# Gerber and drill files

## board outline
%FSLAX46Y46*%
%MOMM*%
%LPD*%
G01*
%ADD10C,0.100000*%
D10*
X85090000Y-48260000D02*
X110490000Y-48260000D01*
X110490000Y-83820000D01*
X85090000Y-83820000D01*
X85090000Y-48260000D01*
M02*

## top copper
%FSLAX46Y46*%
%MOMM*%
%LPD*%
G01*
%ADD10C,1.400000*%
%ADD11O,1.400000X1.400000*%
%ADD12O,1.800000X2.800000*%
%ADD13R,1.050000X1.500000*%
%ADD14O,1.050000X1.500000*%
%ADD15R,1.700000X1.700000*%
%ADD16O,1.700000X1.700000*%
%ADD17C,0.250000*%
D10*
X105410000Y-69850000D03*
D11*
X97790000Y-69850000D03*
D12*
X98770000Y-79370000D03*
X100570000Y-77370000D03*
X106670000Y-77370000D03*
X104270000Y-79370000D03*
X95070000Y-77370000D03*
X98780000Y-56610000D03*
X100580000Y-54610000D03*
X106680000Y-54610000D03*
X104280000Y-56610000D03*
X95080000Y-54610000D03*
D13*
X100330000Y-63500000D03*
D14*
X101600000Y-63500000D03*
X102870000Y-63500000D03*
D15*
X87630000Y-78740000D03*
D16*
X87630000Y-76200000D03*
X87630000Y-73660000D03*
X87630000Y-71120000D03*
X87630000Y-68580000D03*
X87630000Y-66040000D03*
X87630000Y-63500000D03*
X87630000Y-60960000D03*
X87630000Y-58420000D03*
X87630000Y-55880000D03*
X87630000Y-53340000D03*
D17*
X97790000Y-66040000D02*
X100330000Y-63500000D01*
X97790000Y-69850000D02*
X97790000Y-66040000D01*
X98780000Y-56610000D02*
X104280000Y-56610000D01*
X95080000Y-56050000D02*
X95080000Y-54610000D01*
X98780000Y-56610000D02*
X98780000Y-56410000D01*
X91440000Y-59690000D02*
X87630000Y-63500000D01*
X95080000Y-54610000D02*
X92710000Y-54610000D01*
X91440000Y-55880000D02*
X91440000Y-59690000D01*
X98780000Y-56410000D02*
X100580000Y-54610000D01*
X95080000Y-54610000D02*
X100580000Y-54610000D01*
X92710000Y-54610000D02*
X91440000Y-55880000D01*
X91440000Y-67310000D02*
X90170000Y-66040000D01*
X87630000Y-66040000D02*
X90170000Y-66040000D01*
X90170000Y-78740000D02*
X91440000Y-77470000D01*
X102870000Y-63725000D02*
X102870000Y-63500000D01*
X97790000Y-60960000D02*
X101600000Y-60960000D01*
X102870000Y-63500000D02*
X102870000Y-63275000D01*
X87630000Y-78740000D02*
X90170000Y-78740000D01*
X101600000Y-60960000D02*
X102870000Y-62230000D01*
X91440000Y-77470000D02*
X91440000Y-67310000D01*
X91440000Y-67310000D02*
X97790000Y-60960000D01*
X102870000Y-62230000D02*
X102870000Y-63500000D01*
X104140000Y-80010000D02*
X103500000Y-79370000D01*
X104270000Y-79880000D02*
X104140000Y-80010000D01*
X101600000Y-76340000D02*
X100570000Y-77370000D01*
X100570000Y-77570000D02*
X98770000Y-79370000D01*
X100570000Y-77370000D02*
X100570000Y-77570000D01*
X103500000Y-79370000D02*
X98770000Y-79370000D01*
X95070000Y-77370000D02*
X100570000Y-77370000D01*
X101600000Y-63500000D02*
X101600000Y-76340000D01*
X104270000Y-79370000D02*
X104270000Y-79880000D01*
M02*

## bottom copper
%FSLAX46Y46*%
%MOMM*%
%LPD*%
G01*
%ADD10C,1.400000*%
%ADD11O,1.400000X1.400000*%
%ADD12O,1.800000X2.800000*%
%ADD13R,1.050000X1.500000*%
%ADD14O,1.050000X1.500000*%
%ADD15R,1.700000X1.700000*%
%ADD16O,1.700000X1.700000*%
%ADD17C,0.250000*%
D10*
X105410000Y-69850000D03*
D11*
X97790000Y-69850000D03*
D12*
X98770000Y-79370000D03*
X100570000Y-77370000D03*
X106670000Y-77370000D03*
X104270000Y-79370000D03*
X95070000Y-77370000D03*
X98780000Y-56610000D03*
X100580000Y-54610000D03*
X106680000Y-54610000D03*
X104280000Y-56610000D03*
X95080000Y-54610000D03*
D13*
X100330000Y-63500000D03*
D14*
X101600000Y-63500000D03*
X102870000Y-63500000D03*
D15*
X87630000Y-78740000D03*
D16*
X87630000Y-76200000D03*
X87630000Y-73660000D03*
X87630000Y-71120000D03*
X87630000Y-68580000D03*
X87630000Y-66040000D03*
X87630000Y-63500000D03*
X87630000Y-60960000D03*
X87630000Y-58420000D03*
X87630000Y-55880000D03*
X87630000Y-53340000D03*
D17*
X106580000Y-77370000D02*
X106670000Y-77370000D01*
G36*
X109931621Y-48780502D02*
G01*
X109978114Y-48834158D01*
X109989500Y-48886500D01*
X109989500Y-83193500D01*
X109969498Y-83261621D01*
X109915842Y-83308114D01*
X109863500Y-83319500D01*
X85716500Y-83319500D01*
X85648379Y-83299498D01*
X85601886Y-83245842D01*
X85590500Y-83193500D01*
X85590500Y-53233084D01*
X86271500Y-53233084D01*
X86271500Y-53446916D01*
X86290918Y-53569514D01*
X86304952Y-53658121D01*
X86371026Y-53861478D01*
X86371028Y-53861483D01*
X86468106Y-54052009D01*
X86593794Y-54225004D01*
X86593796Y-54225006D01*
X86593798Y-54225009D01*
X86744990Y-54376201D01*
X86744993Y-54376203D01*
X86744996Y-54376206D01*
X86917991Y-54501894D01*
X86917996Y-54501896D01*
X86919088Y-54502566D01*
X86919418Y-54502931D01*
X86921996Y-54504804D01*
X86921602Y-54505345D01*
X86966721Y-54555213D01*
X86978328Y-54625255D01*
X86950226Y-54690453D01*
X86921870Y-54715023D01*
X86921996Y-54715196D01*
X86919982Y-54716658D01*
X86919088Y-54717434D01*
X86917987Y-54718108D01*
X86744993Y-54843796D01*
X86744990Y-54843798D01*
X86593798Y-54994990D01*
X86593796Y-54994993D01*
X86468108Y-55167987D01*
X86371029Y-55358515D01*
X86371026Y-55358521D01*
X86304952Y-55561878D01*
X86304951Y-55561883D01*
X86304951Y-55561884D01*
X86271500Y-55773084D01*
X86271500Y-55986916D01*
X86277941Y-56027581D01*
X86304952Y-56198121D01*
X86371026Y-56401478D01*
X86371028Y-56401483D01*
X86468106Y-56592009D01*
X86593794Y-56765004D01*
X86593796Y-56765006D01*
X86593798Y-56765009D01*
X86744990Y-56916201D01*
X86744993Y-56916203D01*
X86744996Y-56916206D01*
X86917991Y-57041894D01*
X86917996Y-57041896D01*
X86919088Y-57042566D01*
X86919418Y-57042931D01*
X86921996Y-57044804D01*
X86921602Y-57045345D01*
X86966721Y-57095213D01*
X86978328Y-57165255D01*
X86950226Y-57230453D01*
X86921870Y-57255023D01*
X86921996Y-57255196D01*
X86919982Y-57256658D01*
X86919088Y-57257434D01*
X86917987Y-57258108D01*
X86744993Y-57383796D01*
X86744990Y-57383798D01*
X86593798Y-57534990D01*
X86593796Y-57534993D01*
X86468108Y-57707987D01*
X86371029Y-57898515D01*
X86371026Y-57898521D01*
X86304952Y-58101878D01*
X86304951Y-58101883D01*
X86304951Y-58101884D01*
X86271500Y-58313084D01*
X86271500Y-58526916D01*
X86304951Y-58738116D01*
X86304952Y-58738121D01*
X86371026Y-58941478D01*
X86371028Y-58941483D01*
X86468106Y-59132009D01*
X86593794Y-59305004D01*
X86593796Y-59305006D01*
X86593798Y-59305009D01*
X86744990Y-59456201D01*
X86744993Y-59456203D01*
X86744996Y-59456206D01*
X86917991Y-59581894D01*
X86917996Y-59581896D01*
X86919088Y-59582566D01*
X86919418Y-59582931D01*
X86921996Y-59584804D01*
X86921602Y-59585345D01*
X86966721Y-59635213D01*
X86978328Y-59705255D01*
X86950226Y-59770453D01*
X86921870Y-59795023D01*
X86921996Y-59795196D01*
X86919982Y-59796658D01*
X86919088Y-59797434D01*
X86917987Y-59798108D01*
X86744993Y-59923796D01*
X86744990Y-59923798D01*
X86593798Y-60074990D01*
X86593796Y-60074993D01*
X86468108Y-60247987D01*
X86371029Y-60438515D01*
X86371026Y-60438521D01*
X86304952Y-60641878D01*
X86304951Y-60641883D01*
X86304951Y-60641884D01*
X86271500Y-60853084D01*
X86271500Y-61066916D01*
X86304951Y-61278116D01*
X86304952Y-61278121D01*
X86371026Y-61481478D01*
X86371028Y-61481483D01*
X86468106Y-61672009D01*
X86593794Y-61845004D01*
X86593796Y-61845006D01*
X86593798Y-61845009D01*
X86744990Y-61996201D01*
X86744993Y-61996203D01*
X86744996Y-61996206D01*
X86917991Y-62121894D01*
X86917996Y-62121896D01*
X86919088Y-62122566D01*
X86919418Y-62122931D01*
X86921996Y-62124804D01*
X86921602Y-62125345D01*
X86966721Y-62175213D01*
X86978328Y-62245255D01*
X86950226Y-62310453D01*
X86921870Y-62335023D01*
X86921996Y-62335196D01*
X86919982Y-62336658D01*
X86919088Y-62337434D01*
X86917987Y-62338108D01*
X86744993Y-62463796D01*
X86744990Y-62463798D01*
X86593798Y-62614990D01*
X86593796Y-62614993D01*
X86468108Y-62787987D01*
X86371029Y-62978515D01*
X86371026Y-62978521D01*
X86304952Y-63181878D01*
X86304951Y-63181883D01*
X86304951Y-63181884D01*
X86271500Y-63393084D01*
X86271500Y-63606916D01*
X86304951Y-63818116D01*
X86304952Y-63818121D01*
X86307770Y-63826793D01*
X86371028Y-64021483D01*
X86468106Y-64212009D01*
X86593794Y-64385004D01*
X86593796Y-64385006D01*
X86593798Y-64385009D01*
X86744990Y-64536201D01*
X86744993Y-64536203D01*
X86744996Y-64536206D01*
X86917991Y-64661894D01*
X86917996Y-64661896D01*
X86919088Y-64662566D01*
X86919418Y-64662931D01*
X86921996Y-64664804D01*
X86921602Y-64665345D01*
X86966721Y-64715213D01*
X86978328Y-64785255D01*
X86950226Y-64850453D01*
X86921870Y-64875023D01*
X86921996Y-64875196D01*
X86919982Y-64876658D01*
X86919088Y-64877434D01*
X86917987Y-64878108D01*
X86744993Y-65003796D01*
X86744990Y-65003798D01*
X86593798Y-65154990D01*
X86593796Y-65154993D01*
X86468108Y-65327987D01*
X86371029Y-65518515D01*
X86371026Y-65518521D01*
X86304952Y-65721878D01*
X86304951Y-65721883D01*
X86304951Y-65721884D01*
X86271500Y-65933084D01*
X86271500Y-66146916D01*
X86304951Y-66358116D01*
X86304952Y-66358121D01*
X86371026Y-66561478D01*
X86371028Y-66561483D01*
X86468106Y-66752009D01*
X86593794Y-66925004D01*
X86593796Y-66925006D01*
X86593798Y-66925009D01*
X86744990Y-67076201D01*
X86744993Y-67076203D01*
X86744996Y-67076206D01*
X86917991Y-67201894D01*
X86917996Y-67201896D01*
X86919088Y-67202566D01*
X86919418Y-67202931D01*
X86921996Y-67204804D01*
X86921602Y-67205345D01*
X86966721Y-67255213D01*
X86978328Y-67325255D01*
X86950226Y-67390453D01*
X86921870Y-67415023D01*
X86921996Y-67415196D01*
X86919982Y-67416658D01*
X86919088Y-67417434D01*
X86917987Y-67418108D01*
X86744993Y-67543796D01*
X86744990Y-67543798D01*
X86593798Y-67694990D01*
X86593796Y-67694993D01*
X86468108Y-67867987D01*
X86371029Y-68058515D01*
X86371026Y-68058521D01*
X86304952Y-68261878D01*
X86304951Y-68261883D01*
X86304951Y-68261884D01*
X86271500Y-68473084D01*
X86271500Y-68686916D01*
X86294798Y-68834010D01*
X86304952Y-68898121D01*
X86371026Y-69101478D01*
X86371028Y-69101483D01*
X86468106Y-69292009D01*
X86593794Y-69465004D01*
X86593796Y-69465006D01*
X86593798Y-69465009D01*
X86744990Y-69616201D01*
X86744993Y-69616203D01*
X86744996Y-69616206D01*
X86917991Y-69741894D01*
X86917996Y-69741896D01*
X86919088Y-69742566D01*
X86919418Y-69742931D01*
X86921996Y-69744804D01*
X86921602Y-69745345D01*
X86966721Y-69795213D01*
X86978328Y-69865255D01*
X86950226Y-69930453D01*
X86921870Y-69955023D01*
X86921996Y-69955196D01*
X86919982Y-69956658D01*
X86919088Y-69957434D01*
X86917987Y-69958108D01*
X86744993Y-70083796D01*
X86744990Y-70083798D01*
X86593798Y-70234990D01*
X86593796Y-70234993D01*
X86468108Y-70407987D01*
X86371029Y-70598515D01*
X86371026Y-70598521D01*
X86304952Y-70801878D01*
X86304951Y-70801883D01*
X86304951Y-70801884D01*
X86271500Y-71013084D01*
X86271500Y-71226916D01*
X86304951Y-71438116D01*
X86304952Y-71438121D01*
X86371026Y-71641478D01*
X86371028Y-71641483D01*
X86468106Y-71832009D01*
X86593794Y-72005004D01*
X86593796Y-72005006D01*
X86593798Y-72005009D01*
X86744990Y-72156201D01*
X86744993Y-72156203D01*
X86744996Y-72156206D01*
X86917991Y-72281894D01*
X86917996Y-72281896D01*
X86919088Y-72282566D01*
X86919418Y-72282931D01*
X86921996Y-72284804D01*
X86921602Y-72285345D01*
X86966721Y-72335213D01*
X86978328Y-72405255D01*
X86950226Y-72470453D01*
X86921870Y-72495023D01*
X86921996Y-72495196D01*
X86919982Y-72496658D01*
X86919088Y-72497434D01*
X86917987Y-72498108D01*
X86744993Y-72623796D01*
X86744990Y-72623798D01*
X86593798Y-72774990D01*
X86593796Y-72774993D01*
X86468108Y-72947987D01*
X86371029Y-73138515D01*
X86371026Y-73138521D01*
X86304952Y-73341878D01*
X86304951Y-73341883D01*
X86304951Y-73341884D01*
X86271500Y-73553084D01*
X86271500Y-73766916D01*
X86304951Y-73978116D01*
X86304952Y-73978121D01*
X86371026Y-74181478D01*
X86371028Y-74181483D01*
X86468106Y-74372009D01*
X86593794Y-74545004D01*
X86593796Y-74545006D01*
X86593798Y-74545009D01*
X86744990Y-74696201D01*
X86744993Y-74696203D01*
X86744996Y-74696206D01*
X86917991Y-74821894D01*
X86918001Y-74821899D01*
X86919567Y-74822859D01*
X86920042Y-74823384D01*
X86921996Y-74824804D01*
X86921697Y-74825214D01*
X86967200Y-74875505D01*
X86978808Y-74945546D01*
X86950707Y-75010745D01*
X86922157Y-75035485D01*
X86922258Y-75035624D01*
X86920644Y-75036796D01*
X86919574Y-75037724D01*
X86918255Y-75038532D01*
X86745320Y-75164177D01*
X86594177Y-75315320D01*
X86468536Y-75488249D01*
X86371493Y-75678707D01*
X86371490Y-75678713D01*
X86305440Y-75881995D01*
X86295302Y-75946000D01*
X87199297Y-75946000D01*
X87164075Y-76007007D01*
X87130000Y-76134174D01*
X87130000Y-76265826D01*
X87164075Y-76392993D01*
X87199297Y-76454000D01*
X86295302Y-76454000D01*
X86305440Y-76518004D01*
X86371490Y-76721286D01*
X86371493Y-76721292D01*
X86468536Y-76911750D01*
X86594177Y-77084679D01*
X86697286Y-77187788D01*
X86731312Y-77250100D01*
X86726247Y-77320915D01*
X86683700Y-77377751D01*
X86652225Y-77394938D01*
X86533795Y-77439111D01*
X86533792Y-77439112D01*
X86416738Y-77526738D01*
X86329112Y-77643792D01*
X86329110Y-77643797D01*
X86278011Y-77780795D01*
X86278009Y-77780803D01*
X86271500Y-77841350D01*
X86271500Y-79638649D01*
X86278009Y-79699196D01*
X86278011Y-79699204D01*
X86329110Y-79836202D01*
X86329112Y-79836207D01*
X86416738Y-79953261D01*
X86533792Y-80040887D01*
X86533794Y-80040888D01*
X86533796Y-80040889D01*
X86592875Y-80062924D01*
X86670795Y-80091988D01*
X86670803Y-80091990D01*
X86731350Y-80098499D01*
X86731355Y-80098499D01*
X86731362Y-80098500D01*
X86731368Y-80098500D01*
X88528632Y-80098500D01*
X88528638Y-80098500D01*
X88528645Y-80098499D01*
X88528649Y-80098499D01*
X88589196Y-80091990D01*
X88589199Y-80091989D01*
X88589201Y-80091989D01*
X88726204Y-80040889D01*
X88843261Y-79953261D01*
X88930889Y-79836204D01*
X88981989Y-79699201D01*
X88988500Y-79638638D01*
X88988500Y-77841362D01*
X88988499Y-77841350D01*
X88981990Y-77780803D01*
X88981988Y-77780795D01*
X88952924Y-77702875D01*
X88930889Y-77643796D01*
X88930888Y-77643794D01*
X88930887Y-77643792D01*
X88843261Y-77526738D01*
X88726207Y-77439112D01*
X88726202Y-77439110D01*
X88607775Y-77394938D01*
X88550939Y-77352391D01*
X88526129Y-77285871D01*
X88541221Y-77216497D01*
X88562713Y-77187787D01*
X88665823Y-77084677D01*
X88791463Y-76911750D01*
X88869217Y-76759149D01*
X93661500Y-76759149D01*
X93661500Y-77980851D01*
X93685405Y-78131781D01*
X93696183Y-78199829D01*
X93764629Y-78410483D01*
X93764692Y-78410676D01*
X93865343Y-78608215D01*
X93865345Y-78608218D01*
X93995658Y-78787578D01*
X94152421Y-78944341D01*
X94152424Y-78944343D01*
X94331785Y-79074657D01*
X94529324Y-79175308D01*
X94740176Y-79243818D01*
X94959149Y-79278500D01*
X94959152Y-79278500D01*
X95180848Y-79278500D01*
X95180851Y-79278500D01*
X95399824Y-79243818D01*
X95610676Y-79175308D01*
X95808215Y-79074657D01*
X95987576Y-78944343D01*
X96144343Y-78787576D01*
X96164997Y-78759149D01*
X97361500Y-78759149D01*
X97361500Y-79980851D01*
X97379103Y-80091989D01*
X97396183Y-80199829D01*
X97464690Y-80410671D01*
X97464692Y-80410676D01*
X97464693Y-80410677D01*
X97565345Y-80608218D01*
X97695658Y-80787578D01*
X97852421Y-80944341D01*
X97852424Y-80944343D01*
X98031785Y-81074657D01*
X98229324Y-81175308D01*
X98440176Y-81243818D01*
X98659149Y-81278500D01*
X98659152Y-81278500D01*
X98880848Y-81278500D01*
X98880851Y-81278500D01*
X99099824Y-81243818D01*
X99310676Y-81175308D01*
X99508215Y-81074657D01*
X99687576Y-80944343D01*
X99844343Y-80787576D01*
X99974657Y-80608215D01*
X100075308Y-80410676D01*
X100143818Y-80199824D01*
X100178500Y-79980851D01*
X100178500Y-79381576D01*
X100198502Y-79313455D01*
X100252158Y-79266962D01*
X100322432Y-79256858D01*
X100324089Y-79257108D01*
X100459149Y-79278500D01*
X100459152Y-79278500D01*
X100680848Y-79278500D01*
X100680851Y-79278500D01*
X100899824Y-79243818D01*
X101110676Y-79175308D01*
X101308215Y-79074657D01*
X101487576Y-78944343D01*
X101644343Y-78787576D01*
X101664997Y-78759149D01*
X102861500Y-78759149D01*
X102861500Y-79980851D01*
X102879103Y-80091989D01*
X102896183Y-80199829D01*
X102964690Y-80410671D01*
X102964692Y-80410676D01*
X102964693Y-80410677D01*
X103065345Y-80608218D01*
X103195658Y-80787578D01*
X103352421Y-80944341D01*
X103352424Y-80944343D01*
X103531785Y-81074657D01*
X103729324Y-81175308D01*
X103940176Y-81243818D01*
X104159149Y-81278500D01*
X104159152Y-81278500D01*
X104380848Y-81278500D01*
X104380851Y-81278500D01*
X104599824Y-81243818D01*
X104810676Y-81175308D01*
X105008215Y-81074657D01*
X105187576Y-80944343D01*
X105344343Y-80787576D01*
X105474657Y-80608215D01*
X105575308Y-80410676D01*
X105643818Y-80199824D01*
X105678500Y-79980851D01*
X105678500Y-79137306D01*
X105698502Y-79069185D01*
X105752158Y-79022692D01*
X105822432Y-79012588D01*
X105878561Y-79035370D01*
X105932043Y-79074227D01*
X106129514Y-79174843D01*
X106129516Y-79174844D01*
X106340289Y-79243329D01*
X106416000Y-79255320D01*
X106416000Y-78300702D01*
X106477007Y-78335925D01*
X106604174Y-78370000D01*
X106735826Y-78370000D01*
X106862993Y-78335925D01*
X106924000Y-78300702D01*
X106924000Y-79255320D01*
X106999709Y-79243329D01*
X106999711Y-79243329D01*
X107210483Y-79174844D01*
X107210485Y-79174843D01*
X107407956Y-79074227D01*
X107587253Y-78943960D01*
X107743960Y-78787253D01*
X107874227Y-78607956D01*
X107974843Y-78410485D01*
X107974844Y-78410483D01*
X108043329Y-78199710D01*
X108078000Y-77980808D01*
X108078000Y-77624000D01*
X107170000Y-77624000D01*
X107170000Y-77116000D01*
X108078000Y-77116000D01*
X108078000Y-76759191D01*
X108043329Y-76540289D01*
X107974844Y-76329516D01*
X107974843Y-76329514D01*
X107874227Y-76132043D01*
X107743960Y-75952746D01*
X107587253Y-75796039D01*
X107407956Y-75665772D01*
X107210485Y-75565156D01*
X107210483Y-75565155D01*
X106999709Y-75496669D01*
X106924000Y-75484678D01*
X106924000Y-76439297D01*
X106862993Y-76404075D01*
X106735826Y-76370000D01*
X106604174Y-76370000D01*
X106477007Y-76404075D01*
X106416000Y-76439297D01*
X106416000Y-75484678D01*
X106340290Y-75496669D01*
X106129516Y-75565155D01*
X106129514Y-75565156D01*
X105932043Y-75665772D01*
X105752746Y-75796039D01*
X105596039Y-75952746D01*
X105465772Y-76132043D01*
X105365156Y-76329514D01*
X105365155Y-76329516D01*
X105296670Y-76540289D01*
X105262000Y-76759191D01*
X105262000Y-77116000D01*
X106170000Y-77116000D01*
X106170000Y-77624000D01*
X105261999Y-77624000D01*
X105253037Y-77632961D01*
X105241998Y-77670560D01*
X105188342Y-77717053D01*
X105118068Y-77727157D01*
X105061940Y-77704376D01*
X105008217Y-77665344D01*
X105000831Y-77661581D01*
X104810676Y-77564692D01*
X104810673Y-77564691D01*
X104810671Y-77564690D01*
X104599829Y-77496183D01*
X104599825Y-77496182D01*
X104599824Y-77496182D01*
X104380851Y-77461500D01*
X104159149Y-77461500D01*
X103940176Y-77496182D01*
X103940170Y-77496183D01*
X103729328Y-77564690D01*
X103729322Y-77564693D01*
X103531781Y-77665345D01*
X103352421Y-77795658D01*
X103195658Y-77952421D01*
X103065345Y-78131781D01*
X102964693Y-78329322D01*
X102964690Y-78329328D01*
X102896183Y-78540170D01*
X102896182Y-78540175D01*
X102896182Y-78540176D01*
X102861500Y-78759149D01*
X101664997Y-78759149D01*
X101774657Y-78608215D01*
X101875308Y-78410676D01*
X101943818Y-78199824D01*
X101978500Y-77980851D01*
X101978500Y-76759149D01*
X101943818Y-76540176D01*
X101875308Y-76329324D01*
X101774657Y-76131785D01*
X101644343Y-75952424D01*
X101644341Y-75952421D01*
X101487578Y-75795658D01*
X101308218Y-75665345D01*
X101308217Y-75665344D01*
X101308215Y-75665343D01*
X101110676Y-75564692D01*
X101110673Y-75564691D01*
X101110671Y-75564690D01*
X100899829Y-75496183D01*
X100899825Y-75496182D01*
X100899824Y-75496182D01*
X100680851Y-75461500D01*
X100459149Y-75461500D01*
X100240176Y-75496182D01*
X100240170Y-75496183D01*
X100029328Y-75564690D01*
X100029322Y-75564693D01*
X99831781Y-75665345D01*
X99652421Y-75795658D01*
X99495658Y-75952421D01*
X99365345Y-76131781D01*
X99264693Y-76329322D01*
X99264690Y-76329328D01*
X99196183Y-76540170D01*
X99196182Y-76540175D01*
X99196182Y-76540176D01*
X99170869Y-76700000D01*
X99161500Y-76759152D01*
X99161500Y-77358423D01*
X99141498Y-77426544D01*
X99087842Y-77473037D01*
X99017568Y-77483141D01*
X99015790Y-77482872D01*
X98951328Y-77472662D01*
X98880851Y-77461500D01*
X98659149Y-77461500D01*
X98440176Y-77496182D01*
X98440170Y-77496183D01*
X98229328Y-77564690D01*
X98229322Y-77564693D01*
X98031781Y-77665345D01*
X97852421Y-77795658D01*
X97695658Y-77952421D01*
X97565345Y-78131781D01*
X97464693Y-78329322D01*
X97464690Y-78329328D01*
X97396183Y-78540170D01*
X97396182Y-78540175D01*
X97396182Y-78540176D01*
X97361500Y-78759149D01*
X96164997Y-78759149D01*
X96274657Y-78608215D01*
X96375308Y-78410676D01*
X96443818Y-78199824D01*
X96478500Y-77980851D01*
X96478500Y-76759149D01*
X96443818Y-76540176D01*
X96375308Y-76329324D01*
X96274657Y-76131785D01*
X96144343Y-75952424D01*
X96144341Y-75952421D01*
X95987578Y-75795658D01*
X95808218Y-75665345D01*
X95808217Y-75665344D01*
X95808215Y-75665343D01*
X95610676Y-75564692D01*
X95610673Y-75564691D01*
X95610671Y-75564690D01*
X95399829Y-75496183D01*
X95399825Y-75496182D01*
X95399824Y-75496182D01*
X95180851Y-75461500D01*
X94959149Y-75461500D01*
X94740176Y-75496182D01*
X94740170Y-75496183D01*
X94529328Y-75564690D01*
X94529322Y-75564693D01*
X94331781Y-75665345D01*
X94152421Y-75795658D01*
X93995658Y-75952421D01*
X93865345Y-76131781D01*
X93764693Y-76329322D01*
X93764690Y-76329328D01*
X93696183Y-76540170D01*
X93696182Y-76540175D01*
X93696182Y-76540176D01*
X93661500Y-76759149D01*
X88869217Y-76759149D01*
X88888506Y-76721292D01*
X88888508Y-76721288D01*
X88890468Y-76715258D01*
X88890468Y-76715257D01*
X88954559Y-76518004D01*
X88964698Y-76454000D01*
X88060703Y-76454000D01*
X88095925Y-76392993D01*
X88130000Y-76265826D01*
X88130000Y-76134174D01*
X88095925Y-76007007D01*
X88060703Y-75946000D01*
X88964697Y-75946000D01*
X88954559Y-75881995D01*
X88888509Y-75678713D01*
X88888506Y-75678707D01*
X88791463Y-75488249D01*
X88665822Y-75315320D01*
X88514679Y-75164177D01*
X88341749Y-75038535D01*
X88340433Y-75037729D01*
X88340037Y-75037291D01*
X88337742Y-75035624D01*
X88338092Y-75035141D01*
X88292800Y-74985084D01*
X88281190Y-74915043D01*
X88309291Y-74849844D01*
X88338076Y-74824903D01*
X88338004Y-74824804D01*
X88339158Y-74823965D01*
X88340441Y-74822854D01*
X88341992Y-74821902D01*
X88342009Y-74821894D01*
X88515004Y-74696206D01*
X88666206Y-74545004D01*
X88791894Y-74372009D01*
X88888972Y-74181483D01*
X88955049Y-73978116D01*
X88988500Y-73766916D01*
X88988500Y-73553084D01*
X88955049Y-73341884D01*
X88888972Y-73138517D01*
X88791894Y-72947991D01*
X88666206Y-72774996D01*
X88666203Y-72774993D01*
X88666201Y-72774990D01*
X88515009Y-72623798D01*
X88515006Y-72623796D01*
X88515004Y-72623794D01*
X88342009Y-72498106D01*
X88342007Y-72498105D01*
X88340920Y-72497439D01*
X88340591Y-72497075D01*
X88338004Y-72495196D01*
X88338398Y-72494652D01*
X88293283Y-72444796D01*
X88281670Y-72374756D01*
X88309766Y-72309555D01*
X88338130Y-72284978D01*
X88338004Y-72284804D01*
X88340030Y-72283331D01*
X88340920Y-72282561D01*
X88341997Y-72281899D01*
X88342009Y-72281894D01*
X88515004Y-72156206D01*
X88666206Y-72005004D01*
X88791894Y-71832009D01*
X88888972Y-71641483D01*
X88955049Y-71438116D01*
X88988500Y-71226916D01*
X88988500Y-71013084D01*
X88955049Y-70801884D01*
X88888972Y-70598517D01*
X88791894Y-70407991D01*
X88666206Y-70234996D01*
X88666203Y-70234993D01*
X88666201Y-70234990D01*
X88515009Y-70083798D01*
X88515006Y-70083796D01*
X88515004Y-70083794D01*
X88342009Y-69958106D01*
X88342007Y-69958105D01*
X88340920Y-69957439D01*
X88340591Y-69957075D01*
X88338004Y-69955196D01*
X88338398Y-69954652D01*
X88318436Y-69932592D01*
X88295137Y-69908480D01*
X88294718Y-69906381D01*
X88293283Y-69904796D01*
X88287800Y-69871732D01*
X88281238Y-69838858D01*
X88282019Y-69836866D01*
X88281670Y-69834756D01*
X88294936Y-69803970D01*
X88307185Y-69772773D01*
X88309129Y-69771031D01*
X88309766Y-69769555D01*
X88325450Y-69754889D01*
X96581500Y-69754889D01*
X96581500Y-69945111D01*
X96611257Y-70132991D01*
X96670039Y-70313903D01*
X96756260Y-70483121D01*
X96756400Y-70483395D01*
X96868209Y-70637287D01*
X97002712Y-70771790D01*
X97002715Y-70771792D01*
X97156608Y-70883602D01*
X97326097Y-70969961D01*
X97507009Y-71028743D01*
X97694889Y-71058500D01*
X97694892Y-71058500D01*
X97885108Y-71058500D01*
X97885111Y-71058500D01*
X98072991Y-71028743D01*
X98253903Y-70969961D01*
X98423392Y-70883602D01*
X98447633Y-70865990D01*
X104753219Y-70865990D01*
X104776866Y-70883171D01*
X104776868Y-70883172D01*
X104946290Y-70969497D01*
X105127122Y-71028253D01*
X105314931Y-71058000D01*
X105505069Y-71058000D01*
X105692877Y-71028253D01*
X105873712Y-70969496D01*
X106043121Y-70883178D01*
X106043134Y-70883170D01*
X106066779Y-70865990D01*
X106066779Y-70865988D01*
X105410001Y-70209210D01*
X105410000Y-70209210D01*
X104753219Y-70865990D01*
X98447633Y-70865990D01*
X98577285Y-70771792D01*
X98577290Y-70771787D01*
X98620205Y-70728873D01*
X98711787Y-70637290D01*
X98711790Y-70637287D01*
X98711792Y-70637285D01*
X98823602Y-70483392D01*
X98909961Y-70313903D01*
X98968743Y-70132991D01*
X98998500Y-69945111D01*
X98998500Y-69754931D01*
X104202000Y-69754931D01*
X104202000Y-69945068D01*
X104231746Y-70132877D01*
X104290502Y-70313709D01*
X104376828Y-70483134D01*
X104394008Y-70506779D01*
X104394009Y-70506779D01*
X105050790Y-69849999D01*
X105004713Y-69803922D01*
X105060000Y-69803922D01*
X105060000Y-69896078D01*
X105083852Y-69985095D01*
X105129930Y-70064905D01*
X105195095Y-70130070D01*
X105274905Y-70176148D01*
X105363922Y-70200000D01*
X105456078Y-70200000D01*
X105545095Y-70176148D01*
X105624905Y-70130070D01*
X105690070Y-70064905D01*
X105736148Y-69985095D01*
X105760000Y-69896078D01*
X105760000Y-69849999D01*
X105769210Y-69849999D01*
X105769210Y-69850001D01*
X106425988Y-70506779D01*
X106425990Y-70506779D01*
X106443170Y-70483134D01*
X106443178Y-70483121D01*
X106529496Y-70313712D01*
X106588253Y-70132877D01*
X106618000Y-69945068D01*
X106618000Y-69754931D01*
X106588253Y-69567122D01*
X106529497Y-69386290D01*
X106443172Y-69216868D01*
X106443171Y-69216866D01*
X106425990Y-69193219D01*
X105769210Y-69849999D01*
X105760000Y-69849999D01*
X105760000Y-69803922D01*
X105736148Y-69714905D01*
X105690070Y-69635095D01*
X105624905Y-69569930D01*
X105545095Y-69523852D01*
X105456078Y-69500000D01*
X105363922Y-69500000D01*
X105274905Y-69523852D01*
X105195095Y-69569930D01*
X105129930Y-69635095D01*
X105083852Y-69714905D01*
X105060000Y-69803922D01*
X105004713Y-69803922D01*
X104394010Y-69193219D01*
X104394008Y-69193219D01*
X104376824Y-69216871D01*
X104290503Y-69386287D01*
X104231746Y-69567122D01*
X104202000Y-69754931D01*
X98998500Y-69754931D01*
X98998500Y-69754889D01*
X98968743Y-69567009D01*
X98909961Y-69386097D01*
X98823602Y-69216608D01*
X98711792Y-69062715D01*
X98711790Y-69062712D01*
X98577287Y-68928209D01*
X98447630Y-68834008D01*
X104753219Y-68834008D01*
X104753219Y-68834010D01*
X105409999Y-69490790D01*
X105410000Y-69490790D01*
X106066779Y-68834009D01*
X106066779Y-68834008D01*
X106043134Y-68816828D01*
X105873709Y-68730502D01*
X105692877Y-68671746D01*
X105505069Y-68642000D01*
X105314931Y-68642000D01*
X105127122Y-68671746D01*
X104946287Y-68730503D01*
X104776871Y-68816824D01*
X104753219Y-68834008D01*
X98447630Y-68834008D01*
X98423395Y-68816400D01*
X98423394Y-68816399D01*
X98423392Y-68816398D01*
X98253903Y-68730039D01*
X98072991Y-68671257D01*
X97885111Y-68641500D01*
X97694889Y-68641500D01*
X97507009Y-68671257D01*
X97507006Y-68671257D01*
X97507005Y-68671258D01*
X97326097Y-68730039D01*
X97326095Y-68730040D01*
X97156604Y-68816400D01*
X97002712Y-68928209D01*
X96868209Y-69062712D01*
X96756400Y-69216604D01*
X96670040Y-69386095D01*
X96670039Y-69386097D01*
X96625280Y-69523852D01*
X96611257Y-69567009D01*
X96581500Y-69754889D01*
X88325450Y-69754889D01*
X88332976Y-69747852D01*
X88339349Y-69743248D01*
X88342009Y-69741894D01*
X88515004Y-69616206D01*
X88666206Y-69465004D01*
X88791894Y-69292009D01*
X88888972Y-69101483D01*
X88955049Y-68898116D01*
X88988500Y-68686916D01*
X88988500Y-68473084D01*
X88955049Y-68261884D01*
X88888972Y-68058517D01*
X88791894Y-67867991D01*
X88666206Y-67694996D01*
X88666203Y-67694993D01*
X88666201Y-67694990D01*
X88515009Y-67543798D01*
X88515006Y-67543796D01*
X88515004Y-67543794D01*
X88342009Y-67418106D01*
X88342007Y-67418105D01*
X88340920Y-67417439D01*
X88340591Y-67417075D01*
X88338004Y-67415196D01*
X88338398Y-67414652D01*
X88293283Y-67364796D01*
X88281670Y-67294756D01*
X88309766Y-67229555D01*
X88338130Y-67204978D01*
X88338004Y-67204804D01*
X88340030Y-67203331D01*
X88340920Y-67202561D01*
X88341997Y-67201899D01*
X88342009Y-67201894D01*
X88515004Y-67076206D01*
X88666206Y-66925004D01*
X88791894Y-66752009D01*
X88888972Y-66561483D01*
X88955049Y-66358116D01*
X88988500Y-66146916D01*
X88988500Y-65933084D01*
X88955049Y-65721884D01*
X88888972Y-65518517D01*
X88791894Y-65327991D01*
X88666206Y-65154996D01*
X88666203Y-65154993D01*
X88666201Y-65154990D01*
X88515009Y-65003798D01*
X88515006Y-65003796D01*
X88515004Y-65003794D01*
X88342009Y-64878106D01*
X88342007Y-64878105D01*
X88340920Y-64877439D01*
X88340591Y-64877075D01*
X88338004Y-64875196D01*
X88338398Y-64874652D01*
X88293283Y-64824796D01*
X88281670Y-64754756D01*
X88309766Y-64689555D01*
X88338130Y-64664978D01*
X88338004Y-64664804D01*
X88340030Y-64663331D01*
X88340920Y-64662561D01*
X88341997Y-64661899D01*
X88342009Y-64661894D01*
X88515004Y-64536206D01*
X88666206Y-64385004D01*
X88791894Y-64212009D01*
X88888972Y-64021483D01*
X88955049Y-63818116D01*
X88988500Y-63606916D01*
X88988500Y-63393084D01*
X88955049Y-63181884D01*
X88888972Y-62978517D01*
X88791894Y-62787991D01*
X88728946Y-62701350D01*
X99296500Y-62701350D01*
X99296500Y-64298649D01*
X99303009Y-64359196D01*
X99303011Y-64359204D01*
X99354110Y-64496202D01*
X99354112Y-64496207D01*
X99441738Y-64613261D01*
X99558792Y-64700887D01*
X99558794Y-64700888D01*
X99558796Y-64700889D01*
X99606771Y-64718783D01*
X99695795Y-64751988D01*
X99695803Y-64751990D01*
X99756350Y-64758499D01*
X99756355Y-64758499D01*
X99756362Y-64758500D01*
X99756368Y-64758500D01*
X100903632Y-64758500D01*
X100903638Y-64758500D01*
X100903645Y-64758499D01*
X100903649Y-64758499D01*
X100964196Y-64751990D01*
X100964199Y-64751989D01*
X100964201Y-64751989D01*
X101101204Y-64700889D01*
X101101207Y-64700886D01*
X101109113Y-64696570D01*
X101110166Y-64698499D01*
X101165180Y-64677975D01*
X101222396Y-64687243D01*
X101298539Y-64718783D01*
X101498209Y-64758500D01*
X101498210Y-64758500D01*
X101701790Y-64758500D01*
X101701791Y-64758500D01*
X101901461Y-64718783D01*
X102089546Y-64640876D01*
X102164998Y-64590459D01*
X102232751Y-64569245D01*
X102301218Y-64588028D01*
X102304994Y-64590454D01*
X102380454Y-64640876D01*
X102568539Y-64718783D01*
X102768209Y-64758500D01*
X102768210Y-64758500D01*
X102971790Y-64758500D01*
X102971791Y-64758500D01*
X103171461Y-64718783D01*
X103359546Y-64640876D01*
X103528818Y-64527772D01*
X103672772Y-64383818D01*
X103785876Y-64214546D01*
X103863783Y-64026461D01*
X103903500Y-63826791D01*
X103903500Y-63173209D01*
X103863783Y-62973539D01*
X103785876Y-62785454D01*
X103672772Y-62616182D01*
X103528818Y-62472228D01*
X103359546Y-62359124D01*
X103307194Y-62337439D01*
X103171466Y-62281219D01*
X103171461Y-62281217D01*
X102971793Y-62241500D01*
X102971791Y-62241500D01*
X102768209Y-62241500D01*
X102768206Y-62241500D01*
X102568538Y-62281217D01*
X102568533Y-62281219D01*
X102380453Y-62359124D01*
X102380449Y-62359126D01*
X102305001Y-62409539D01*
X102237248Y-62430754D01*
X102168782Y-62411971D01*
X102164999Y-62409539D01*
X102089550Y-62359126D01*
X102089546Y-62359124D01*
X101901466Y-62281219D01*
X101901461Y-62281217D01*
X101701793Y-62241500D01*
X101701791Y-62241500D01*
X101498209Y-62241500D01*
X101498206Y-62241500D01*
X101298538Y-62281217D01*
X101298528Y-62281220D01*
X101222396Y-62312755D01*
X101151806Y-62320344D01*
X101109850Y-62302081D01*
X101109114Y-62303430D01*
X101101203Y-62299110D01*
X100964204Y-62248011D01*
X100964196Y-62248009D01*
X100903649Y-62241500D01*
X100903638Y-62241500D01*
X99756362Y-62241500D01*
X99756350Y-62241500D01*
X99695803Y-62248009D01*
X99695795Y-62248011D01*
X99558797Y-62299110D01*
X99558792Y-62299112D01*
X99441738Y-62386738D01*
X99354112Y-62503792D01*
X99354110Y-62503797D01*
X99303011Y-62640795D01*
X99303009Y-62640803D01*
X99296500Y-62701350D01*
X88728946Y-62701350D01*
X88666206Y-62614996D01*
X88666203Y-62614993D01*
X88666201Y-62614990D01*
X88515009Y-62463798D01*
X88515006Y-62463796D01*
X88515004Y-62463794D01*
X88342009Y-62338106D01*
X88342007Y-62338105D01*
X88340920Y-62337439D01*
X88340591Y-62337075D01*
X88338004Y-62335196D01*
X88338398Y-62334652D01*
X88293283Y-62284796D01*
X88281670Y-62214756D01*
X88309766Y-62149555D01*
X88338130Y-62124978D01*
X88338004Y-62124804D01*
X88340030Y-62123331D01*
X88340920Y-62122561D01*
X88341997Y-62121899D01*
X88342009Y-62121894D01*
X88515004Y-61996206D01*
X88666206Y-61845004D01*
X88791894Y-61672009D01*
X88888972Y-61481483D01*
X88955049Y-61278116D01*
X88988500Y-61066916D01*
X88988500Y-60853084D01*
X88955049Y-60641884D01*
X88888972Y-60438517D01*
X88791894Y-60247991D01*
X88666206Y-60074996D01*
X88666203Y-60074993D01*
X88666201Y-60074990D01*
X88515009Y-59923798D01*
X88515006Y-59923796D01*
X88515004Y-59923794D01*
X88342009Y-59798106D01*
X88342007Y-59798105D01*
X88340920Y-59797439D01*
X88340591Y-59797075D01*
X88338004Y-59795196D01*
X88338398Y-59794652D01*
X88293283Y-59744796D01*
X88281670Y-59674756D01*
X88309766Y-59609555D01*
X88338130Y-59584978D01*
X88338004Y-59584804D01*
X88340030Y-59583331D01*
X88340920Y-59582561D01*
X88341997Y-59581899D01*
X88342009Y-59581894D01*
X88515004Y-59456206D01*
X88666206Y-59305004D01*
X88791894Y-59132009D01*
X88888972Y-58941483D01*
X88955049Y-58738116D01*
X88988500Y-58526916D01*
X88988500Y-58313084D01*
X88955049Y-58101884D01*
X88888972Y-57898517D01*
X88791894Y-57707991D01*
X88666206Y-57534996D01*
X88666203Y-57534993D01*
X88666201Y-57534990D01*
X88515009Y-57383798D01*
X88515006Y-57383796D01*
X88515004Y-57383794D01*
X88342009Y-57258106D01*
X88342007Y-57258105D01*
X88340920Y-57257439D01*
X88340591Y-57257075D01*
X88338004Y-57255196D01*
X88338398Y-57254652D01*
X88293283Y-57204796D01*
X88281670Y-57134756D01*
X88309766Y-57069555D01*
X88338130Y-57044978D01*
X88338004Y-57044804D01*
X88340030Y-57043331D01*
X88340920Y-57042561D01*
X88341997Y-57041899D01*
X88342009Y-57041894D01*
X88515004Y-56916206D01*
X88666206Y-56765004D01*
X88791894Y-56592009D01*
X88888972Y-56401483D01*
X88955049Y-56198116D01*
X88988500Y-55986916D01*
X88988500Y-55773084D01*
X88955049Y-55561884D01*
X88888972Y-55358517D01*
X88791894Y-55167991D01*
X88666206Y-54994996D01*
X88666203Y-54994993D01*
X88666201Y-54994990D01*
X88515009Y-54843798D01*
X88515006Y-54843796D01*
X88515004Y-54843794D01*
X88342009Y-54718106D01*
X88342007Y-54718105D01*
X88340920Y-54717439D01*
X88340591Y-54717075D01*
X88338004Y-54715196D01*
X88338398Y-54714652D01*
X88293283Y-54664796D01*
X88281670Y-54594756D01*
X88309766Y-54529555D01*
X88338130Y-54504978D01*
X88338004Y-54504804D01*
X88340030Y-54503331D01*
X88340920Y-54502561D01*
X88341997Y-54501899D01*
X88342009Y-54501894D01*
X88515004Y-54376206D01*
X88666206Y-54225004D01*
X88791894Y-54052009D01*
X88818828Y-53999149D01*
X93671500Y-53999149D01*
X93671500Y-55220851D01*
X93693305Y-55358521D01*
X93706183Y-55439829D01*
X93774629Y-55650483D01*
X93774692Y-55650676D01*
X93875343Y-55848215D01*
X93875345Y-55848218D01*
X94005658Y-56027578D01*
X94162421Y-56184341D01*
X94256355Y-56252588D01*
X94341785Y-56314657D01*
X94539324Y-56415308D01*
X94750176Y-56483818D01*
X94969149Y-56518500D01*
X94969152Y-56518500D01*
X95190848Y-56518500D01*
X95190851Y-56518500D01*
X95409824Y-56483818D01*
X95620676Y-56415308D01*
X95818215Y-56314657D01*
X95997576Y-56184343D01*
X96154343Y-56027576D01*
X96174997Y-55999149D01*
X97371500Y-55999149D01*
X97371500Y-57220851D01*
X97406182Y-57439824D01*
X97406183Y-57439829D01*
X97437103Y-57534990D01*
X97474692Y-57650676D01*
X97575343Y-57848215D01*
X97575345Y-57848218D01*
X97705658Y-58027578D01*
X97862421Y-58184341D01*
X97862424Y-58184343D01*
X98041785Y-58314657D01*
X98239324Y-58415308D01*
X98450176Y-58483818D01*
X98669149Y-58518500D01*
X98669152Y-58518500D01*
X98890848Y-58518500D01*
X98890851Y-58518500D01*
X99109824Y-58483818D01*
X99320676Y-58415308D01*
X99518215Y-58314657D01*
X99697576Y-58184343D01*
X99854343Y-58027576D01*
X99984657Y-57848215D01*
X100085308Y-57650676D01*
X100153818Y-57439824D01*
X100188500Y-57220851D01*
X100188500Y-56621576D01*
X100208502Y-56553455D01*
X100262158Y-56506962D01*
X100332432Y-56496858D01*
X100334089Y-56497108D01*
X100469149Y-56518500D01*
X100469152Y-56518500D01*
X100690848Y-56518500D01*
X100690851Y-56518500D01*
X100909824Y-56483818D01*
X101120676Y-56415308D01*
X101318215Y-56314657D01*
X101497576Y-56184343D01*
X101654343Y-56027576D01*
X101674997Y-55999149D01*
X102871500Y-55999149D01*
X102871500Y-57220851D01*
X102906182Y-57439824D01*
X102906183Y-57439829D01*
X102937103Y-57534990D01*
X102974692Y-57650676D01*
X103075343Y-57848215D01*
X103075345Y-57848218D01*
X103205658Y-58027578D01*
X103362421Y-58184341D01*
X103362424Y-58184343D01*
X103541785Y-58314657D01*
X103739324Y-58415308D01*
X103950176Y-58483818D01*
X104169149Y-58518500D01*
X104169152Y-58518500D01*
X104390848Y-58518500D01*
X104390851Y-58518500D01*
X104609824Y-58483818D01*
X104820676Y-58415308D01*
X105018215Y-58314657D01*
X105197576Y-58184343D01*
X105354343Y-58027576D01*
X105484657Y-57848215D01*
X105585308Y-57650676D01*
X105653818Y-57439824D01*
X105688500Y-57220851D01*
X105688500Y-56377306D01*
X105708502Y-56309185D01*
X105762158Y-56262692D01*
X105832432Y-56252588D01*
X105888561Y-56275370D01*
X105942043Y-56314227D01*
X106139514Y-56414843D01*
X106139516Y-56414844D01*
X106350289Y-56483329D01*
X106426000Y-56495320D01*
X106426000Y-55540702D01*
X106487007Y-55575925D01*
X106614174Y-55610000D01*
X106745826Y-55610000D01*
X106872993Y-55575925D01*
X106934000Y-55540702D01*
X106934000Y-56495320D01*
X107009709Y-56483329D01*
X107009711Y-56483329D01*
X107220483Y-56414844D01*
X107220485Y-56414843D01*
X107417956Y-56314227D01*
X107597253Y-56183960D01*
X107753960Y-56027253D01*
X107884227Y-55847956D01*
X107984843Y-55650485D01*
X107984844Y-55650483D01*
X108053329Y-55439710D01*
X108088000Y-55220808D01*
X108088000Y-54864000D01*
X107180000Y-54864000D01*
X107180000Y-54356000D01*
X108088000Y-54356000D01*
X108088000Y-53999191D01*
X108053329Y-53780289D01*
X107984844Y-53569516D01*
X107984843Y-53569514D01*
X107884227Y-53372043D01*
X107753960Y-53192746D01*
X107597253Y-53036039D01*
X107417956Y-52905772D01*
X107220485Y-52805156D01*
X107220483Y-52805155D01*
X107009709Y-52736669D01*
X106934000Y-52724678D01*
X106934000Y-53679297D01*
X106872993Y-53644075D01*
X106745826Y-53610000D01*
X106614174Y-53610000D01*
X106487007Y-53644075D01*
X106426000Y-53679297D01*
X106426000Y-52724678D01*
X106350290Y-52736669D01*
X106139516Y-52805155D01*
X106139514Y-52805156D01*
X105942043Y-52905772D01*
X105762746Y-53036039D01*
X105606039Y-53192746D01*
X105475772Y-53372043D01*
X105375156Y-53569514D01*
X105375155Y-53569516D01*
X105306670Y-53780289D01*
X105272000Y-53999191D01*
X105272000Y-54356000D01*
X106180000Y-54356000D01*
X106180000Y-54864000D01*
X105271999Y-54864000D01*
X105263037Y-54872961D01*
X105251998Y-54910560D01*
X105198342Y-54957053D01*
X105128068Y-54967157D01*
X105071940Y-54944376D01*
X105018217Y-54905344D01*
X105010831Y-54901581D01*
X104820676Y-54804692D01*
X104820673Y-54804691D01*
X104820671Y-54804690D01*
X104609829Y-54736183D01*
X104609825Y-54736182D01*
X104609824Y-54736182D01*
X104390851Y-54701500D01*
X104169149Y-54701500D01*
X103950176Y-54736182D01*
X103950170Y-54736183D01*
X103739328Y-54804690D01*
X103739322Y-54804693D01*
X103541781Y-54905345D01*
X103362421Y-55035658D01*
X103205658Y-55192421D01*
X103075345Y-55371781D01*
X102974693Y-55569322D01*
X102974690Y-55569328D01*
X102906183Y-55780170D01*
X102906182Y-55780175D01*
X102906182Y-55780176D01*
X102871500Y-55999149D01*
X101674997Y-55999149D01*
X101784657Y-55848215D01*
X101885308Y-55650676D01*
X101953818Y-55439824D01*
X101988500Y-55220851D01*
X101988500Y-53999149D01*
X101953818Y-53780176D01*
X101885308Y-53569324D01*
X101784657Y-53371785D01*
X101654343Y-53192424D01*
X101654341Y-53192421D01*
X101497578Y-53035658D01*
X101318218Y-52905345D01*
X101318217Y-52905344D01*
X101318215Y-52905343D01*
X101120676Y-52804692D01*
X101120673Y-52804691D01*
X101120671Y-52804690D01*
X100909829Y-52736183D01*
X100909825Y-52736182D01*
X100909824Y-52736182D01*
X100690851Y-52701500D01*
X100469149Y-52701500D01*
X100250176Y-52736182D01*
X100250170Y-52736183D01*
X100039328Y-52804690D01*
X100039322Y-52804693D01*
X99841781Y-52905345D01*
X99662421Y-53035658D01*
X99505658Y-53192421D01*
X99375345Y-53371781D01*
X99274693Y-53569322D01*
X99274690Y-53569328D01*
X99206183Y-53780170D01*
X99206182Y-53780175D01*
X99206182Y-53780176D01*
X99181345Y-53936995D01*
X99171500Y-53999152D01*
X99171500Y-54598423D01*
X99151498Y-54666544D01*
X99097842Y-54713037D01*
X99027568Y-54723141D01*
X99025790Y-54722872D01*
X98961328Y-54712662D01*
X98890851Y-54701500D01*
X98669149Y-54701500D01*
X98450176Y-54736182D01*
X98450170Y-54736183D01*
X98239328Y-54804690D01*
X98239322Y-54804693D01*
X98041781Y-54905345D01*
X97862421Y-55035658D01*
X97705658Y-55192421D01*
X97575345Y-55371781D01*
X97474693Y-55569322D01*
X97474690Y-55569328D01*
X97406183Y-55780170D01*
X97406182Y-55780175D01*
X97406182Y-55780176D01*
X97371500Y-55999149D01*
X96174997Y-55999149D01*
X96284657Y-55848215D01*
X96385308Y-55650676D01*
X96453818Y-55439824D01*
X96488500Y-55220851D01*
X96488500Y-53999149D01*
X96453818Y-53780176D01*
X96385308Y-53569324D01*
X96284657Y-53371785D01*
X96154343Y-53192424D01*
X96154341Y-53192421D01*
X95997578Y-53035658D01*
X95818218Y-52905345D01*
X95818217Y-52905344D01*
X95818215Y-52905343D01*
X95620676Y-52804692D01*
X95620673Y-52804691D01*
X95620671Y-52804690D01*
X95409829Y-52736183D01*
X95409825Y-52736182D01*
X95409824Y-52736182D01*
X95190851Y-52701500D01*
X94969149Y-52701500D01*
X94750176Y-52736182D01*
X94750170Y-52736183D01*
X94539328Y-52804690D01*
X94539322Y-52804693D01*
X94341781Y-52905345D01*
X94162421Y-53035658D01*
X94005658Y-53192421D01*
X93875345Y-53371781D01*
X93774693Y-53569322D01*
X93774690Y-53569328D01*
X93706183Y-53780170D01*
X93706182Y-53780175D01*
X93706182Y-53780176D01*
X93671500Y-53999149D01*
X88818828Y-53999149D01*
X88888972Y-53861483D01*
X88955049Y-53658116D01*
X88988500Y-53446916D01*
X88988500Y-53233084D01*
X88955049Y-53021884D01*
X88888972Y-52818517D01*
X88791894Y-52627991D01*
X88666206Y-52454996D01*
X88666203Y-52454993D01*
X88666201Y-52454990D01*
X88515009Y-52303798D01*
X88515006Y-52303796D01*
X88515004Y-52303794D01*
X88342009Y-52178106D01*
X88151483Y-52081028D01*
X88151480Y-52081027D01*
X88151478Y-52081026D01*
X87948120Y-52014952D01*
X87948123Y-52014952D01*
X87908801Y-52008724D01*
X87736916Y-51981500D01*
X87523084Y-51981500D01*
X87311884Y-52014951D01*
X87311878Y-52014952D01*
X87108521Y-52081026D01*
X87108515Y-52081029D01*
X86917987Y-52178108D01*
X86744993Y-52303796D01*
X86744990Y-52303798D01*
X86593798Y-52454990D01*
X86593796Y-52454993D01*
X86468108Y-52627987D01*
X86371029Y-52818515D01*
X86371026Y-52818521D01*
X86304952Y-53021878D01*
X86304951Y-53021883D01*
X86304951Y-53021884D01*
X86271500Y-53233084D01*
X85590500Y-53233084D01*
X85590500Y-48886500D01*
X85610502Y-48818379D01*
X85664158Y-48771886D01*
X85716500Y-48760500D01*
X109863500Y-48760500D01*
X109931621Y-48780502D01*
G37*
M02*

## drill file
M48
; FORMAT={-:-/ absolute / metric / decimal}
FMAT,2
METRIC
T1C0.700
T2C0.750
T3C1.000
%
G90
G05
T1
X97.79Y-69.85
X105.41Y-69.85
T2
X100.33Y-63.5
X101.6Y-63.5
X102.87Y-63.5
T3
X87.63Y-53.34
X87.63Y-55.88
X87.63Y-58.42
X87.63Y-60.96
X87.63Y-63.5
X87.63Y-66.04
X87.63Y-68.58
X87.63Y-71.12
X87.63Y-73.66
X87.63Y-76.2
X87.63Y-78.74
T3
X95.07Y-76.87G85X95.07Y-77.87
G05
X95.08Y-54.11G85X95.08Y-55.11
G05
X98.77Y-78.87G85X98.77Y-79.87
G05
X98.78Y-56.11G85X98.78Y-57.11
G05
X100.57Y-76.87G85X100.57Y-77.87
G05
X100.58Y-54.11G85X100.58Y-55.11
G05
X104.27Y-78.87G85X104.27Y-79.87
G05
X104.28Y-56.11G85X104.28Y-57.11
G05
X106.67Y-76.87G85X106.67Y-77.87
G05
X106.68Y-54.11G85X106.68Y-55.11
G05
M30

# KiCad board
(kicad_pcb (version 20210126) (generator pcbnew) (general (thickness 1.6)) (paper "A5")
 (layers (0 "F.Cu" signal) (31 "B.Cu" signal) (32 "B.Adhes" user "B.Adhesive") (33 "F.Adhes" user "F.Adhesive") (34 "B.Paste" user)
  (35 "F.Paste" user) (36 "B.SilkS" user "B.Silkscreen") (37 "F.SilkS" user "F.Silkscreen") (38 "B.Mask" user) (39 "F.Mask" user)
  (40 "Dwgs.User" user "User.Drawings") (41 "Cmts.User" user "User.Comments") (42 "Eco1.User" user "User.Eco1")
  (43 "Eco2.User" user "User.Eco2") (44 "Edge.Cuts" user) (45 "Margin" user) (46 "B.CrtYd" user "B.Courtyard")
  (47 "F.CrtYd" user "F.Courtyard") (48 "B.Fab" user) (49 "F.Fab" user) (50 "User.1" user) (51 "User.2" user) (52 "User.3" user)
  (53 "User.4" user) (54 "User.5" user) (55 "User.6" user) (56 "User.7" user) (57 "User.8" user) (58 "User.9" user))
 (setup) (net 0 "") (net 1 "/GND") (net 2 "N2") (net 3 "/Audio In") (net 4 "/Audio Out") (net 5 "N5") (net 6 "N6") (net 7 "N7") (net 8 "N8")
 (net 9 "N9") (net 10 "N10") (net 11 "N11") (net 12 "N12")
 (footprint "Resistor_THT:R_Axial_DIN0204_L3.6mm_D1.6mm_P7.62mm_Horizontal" (layer "F.Cu") (at 105.41 69.85 180)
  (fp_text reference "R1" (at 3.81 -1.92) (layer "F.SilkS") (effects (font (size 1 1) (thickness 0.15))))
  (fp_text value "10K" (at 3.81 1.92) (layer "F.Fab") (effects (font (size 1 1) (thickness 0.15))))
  (pad "1" thru_hole circle (at 0 0 180) (locked) (size 1.4 1.4) (drill 0.7) (layers *.Cu *.Mask) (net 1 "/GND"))
  (pad "2" thru_hole oval (at 7.62 0 180) (locked) (size 1.4 1.4) (drill 0.7) (layers *.Cu *.Mask) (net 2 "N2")))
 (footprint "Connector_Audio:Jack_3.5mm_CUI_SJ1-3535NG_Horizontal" (layer "F.Cu") (at 106.67 77.37 -90)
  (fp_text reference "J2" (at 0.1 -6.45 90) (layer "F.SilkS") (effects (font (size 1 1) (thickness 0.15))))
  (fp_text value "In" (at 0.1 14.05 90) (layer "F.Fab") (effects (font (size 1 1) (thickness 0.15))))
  (pad "R" thru_hole oval (at 2 7.9 270) (locked) (size 2.8 1.8) (drill oval 2 1) (layers *.Cu *.Mask) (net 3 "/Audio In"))
  (pad "RN" thru_hole oval (at 0 6.1 270) (locked) (size 2.8 1.8) (drill oval 2 1) (layers *.Cu *.Mask) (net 3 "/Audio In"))
  (pad "S" thru_hole oval (at 0 0 270) (locked) (size 2.8 1.8) (drill oval 2 1) (layers *.Cu *.Mask) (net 1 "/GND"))
  (pad "T" thru_hole oval (at 2 2.4 270) (locked) (size 2.8 1.8) (drill oval 2 1) (layers *.Cu *.Mask) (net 3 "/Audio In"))
  (pad "TN" thru_hole oval (at 0 11.6 270) (locked) (size 2.8 1.8) (drill oval 2 1) (layers *.Cu *.Mask) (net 3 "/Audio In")))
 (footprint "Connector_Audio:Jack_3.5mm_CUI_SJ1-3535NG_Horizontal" (layer "F.Cu") (at 106.68 54.61 -90)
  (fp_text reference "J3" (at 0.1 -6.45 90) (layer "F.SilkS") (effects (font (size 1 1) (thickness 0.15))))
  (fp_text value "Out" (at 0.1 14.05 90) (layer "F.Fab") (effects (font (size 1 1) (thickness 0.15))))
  (pad "R" thru_hole oval (at 2 7.9 270) (locked) (size 2.8 1.8) (drill oval 2 1) (layers *.Cu *.Mask) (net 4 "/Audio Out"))
  (pad "RN" thru_hole oval (at 0 6.1 270) (locked) (size 2.8 1.8) (drill oval 2 1) (layers *.Cu *.Mask) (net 4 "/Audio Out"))
  (pad "S" thru_hole oval (at 0 0 270) (locked) (size 2.8 1.8) (drill oval 2 1) (layers *.Cu *.Mask) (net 1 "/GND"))
  (pad "T" thru_hole oval (at 2 2.4 270) (locked) (size 2.8 1.8) (drill oval 2 1) (layers *.Cu *.Mask) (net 4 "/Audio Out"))
  (pad "TN" thru_hole oval (at 0 11.6 270) (locked) (size 2.8 1.8) (drill oval 2 1) (layers *.Cu *.Mask) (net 4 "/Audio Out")))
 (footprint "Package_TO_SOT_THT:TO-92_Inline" (layer "F.Cu") (at 100.33 63.5)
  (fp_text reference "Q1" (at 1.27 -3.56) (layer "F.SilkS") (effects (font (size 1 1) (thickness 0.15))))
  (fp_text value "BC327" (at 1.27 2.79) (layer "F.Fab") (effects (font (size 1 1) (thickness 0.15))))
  (pad "1" thru_hole rect (at 0 0) (locked) (size 1.05 1.5) (drill 0.75) (layers *.Cu *.Mask) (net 2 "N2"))
  (pad "2" thru_hole oval (at 1.27 0) (locked) (size 1.05 1.5) (drill 0.75) (layers *.Cu *.Mask) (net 3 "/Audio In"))
  (pad "3" thru_hole oval (at 2.54 0) (locked) (size 1.05 1.5) (drill 0.75) (layers *.Cu *.Mask) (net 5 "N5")))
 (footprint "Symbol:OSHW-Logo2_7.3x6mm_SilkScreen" (layer "F.Cu") (at 92.71 64.77 90)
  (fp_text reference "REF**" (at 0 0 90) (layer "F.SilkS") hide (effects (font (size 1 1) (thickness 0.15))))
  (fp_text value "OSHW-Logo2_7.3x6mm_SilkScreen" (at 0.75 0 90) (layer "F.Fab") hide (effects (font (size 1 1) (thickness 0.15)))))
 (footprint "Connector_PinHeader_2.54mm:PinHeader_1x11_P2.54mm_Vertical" (layer "F.Cu") (at 87.63 78.74 180)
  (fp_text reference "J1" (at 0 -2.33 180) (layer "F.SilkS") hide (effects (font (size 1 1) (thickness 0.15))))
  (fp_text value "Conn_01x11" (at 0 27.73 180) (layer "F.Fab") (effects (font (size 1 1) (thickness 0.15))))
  (pad "1" thru_hole rect (at 0 0 180) (size 1.7 1.7) (drill 1) (layers *.Cu *.Mask) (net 5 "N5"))
  (pad "2" thru_hole oval (at 0 2.54 180) (size 1.7 1.7) (drill 1) (layers *.Cu *.Mask) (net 1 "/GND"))
  (pad "3" thru_hole oval (at 0 5.08 180) (size 1.7 1.7) (drill 1) (layers *.Cu *.Mask) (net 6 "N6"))
  (pad "4" thru_hole oval (at 0 7.62 180) (size 1.7 1.7) (drill 1) (layers *.Cu *.Mask) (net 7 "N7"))
  (pad "5" thru_hole oval (at 0 10.16 180) (size 1.7 1.7) (drill 1) (layers *.Cu *.Mask) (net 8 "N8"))
  (pad "6" thru_hole oval (at 0 12.7 180) (size 1.7 1.7) (drill 1) (layers *.Cu *.Mask) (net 5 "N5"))
  (pad "7" thru_hole oval (at 0 15.24 180) (size 1.7 1.7) (drill 1) (layers *.Cu *.Mask) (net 4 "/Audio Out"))
  (pad "8" thru_hole oval (at 0 17.78 180) (size 1.7 1.7) (drill 1) (layers *.Cu *.Mask) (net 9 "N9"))
  (pad "9" thru_hole oval (at 0 20.32 180) (size 1.7 1.7) (drill 1) (layers *.Cu *.Mask) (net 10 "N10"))
  (pad "10" thru_hole oval (at 0 22.86 180) (size 1.7 1.7) (drill 1) (layers *.Cu *.Mask) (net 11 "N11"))
  (pad "11" thru_hole oval (at 0 25.4 180) (size 1.7 1.7) (drill 1) (layers *.Cu *.Mask) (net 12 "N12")))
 (gr_rect (start 85.09 48.26) (end 110.49 83.82) (layer "Edge.Cuts") (width 0.1) (fill none))
 (segment (start 106.58 77.37) (end 106.67 77.37) (width 0.25) (layer "B.Cu") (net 1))
 (segment (start 97.79 66.04) (end 100.33 63.5) (width 0.25) (layer "F.Cu") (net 2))
 (segment (start 97.79 69.85) (end 97.79 66.04) (width 0.25) (layer "F.Cu") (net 2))
 (segment (start 98.78 56.61) (end 104.28 56.61) (width 0.25) (layer "F.Cu") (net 4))
 (segment (start 95.08 56.05) (end 95.08 54.61) (width 0.25) (layer "F.Cu") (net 4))
 (segment (start 98.78 56.61) (end 98.78 56.41) (width 0.25) (layer "F.Cu") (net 4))
 (segment (start 91.44 59.69) (end 87.63 63.5) (width 0.25) (layer "F.Cu") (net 4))
 (segment (start 95.08 54.61) (end 92.71 54.61) (width 0.25) (layer "F.Cu") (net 4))
 (segment (start 91.44 55.88) (end 91.44 59.69) (width 0.25) (layer "F.Cu") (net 4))
 (segment (start 98.78 56.41) (end 100.58 54.61) (width 0.25) (layer "F.Cu") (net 4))
 (segment (start 95.08 54.61) (end 100.58 54.61) (width 0.25) (layer "F.Cu") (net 4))
 (segment (start 92.71 54.61) (end 91.44 55.88) (width 0.25) (layer "F.Cu") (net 4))
 (segment (start 91.44 67.31) (end 90.17 66.04) (width 0.25) (layer "F.Cu") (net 5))
 (segment (start 87.63 66.04) (end 90.17 66.04) (width 0.25) (layer "F.Cu") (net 5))
 (segment (start 90.17 78.74) (end 91.44 77.47) (width 0.25) (layer "F.Cu") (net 5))
 (segment (start 102.87 63.725) (end 102.87 63.5) (width 0.25) (layer "F.Cu") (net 5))
 (segment (start 97.79 60.96) (end 101.6 60.96) (width 0.25) (layer "F.Cu") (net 5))
 (segment (start 102.87 63.5) (end 102.87 63.275) (width 0.25) (layer "F.Cu") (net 5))
 (segment (start 87.63 78.74) (end 90.17 78.74) (width 0.25) (layer "F.Cu") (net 5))
 (segment (start 101.6 60.96) (end 102.87 62.23) (width 0.25) (layer "F.Cu") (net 5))
 (segment (start 91.44 77.47) (end 91.44 67.31) (width 0.25) (layer "F.Cu") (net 5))
 (segment (start 91.44 67.31) (end 97.79 60.96) (width 0.25) (layer "F.Cu") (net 5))
 (segment (start 102.87 62.23) (end 102.87 63.5) (width 0.25) (layer "F.Cu") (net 5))
 (segment (start 104.14 80.01) (end 103.5 79.37) (width 0.25) (layer "F.Cu") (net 3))
 (segment (start 104.27 79.88) (end 104.14 80.01) (width 0.25) (layer "F.Cu") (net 3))
 (segment (start 101.6 76.34) (end 100.57 77.37) (width 0.25) (layer "F.Cu") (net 3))
 (segment (start 100.57 77.57) (end 98.77 79.37) (width 0.25) (layer "F.Cu") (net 3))
 (segment (start 100.57 77.37) (end 100.57 77.57) (width 0.25) (layer "F.Cu") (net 3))
 (segment (start 103.5 79.37) (end 98.77 79.37) (width 0.25) (layer "F.Cu") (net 3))
 (segment (start 95.07 77.37) (end 100.57 77.37) (width 0.25) (layer "F.Cu") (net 3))
 (segment (start 101.6 63.5) (end 101.6 76.34) (width 0.25) (layer "F.Cu") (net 3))
 (segment (start 104.27 79.37) (end 104.27 79.88) (width 0.25) (layer "F.Cu") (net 3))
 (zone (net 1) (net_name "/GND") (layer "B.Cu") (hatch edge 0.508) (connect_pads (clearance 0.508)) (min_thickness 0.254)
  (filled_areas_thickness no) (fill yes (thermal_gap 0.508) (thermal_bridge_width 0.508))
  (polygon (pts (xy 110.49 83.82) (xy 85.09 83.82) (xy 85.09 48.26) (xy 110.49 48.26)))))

